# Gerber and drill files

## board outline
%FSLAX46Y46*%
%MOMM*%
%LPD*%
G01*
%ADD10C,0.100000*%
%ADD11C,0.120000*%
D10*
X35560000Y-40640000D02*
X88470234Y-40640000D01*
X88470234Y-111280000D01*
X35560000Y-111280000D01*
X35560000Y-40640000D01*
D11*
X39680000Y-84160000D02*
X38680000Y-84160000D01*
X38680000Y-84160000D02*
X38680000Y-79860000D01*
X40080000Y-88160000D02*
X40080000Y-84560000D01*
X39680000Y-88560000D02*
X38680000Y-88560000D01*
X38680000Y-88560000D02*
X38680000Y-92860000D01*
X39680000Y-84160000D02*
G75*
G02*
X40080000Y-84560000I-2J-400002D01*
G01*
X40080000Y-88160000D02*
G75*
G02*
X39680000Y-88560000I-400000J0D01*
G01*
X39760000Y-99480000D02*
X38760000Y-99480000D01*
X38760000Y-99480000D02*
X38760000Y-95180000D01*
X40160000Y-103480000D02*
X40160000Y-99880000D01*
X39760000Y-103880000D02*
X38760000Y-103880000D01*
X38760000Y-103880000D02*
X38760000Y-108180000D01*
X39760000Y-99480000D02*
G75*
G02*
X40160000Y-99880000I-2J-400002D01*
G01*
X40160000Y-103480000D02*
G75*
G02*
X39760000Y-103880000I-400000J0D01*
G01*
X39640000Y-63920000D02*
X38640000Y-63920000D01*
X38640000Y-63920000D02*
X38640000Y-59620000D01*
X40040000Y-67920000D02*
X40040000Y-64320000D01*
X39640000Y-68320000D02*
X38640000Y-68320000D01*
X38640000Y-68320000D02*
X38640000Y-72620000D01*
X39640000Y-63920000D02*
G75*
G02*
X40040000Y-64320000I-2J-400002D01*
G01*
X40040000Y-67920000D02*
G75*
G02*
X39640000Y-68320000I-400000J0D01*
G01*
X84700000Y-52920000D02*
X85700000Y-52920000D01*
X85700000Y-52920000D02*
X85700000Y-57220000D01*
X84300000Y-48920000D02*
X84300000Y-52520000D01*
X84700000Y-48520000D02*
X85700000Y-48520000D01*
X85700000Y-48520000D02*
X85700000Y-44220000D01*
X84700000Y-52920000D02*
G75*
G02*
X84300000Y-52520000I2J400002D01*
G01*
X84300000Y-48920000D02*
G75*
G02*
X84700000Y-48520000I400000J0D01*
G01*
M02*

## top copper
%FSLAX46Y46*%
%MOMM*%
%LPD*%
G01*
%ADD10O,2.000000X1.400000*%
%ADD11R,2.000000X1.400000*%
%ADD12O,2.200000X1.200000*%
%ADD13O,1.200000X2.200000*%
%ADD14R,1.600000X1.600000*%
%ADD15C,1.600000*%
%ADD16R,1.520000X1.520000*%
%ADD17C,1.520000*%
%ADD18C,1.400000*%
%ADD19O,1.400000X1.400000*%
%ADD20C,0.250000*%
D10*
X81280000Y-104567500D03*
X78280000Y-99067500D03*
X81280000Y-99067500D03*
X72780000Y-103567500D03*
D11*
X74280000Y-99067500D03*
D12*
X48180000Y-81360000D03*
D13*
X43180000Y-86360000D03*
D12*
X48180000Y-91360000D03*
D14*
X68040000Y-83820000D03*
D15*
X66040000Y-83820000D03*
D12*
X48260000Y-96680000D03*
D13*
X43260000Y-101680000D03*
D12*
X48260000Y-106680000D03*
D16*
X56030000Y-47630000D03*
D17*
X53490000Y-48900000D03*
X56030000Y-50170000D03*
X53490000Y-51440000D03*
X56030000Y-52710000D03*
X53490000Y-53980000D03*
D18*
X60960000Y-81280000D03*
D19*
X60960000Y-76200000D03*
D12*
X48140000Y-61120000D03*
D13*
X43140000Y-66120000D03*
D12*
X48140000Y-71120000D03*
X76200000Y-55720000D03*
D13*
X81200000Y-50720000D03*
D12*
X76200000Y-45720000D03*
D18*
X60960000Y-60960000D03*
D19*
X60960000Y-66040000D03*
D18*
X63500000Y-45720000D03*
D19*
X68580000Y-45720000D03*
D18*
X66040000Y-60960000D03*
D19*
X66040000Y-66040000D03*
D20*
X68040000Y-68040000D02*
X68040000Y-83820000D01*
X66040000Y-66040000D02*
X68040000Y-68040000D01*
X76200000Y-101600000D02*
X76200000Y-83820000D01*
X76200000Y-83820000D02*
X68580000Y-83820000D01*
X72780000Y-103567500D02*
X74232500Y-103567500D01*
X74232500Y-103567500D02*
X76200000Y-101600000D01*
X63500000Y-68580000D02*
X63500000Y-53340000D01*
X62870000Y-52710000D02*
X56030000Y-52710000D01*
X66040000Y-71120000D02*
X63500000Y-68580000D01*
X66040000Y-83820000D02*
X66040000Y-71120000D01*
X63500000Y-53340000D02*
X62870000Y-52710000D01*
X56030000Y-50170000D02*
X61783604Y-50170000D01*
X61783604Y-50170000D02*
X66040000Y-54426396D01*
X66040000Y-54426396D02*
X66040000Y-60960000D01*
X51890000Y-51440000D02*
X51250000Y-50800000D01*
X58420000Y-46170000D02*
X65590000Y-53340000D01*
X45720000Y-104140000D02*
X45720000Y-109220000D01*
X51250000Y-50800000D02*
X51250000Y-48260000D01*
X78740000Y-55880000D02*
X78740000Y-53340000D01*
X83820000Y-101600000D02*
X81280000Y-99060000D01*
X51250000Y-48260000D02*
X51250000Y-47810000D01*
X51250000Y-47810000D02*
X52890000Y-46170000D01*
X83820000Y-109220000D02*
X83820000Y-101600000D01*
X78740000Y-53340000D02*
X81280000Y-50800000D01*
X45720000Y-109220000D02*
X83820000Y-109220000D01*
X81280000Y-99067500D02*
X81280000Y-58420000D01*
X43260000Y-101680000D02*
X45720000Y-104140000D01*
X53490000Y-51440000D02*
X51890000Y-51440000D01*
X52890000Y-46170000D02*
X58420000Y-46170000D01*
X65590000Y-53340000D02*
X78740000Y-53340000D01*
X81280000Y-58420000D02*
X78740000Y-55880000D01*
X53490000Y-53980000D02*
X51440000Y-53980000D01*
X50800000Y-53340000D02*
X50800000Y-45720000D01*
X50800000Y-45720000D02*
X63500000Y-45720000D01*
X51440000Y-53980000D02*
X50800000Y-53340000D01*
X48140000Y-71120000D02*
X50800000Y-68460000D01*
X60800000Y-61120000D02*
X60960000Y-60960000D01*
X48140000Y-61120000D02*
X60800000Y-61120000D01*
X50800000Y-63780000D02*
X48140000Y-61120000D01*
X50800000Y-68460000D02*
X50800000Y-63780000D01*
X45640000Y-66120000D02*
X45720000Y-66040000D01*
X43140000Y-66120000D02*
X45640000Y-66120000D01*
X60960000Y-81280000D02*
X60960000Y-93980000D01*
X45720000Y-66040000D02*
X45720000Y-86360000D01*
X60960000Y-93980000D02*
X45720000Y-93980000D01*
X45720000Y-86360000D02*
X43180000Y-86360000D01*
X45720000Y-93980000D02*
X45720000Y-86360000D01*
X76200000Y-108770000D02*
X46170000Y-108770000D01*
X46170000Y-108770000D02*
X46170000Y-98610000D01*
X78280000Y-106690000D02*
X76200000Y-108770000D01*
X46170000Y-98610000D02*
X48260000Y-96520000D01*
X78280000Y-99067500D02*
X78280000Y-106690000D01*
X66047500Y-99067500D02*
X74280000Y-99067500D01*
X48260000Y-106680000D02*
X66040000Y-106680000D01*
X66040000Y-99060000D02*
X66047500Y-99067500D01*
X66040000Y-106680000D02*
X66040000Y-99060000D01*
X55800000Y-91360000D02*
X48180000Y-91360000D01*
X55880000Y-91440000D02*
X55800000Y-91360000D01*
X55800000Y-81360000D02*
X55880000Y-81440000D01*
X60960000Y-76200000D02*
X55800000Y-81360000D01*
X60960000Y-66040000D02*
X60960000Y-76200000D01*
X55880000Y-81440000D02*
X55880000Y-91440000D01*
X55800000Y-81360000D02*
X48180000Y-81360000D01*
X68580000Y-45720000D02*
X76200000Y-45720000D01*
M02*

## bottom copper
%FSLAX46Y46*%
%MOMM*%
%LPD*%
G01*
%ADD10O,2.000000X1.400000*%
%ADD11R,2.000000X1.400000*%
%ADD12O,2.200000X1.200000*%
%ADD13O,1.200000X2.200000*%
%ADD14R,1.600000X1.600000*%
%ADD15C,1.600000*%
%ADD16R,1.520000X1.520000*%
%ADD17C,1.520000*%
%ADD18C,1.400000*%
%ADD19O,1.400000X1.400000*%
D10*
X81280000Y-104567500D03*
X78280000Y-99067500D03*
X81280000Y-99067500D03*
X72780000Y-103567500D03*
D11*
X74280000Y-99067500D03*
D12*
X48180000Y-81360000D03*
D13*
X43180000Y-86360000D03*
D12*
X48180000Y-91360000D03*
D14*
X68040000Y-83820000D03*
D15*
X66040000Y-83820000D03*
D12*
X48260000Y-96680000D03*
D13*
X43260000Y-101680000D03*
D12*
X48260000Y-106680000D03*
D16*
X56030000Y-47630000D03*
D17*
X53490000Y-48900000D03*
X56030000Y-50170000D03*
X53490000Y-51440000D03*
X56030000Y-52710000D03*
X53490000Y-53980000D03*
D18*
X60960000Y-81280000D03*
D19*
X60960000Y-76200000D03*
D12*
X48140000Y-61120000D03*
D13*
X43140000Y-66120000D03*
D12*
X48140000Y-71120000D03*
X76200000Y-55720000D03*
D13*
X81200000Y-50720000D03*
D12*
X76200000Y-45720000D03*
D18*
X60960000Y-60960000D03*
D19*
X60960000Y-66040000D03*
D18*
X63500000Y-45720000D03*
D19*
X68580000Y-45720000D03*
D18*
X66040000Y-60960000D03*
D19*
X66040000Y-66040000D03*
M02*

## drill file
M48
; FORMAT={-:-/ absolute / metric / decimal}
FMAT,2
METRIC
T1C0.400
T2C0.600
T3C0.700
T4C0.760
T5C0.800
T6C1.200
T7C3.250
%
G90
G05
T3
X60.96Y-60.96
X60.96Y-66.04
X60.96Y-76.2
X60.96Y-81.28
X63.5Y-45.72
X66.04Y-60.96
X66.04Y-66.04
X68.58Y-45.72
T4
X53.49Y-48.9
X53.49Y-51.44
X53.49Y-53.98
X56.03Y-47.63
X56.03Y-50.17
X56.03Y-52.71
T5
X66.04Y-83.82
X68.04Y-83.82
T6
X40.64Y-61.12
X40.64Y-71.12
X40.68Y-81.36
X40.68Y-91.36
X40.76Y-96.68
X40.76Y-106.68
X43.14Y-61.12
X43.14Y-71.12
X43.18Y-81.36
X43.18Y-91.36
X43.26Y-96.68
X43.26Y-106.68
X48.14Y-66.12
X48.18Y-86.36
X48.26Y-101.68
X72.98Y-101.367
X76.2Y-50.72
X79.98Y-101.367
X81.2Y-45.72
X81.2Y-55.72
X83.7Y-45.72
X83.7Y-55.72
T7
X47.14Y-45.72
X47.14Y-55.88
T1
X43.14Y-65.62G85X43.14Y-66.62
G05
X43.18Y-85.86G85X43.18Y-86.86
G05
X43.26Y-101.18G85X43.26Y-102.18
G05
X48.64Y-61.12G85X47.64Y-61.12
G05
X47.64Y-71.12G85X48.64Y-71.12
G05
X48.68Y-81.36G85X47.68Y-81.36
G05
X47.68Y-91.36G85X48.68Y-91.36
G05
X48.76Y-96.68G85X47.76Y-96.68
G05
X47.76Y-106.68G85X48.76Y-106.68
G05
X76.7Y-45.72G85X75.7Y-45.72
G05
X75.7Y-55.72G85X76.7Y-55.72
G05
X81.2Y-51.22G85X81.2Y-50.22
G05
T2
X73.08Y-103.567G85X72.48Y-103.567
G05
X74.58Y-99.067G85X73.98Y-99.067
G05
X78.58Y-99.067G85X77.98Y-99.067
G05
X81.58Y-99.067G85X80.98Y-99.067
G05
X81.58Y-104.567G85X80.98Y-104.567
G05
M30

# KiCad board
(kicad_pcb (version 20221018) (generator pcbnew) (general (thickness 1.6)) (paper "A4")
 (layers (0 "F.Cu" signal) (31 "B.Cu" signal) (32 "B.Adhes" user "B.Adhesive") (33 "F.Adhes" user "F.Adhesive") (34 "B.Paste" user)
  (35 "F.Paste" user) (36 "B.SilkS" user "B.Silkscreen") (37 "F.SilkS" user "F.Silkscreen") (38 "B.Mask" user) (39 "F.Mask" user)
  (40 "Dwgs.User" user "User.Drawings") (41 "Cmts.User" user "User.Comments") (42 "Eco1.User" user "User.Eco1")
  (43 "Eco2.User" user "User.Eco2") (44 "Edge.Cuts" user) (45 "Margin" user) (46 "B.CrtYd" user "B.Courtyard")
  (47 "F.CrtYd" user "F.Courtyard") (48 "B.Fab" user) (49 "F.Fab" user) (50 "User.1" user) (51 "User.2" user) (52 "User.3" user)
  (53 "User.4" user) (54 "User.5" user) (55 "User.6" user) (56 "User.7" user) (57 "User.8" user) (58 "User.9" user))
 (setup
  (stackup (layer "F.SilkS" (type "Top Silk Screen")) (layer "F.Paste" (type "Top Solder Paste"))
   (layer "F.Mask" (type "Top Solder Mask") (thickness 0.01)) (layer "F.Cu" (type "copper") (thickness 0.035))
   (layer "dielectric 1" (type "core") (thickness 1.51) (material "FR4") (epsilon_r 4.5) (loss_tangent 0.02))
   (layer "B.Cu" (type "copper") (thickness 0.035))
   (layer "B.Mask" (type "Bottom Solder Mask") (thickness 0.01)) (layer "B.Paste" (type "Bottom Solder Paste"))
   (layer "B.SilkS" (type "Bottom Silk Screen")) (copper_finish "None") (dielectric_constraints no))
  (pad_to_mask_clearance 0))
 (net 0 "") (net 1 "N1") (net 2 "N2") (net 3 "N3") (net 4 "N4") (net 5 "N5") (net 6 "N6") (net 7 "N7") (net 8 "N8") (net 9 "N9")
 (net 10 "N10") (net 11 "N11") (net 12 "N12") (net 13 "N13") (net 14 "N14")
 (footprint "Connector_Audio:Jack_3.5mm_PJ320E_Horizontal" (layer "F.Cu") (at 74.28 99.0675 -90)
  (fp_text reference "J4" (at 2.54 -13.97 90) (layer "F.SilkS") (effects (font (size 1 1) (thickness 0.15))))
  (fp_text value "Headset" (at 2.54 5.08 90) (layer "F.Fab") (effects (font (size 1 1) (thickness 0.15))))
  (pad "" np_thru_hole circle (at 2.3 -5.7 180) (size 1.2 1.2) (drill 1.2) (layers "*.Cu" "*.Mask"))
  (pad "" np_thru_hole circle (at 2.3 1.3 180) (size 1.2 1.2) (drill 1.2) (layers "*.Cu" "*.Mask"))
  (pad "" thru_hole oval (at 5.5 -7 180) (size 2 1.4) (drill oval 1.2 0.6) (layers "*.Cu" "*.Mask"))
  (pad "R1" thru_hole oval (at 0 -4 180) (size 2 1.4) (drill oval 1.2 0.6) (layers "*.Cu" "*.Mask") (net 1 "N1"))
  (pad "R2" thru_hole oval (at 0 -7 180) (size 2 1.4) (drill oval 1.2 0.6) (layers "*.Cu" "*.Mask") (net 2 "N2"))
  (pad "S" thru_hole oval (at 4.5 1.5 180) (size 2 1.4) (drill oval 1.2 0.6) (layers "*.Cu" "*.Mask") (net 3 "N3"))
  (pad "T" thru_hole rect (at 0 0 180) (size 2 1.4) (drill oval 1.2 0.6) (layers "*.Cu" "*.Mask") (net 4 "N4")))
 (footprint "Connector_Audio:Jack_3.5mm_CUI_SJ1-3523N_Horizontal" (layer "F.Cu") (at 43.18 86.36 -90)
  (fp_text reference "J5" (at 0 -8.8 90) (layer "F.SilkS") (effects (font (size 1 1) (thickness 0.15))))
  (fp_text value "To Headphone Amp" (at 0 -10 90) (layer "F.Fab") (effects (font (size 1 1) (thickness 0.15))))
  (fp_line (start -2.2 3.5) (end -2.2 4.5) (stroke (width 0.12) (type solid)) (layer "Edge.Cuts"))
  (fp_line (start -2.2 4.5) (end -6.5 4.5) (stroke (width 0.12) (type solid)) (layer "Edge.Cuts"))
  (fp_line (start 1.8 3.1) (end -1.8 3.1) (stroke (width 0.12) (type solid)) (layer "Edge.Cuts"))
  (fp_line (start 2.2 3.5) (end 2.2 4.5) (stroke (width 0.12) (type solid)) (layer "Edge.Cuts"))
  (fp_line (start 2.2 4.5) (end 6.5 4.5) (stroke (width 0.12) (type solid)) (layer "Edge.Cuts"))
  (fp_arc (start -2.2 3.5) (mid -2.082842 3.217158) (end -1.8 3.1) (stroke (width 0.12) (type solid)) (layer "Edge.Cuts"))
  (fp_arc (start 1.8 3.1) (mid 2.082843 3.217157) (end 2.2 3.5) (stroke (width 0.12) (type solid)) (layer "Edge.Cuts"))
  (pad "" np_thru_hole circle (at -5 0 270) (size 1.2 1.2) (drill 1.2) (layers "*.Cu"))
  (pad "" np_thru_hole circle (at -5 2.5 270) (size 1.2 1.2) (drill 1.2) (layers "*.Cu"))
  (pad "" np_thru_hole circle (at 0 -5 270) (size 1.2 1.2) (drill 1.2) (layers "*.Cu"))
  (pad "" np_thru_hole circle (at 5 0 270) (size 1.2 1.2) (drill 1.2) (layers "*.Cu"))
  (pad "" np_thru_hole circle (at 5 2.5 270) (size 1.2 1.2) (drill 1.2) (layers "*.Cu"))
  (pad "R" thru_hole oval (at -5 -5 270) (size 1.2 2.2) (drill oval 0.4 1.4) (layers "*.Cu" "*.Mask") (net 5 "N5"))
  (pad "S" thru_hole oval (at 0 0 270) (size 2.2 1.2) (drill oval 1.4 0.4) (layers "*.Cu" "*.Mask") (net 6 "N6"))
  (pad "T" thru_hole oval (at 5 -5 90) (size 1.2 2.2) (drill oval 0.4 1.4) (layers "*.Cu" "*.Mask") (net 5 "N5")))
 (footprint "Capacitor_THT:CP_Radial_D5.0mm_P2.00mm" (layer "F.Cu") (at 68.04 83.82 180)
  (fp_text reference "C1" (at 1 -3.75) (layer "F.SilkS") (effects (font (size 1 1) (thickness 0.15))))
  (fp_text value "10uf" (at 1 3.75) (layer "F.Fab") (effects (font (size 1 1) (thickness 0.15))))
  (pad "1" thru_hole rect (at 0 0 180) (size 1.6 1.6) (drill 0.8) (layers "*.Cu" "*.Mask") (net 3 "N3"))
  (pad "2" thru_hole circle (at 2 0 180) (size 1.6 1.6) (drill 0.8) (layers "*.Cu" "*.Mask") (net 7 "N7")))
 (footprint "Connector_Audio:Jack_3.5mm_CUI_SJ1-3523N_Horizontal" (layer "F.Cu") (at 43.26 101.68 -90)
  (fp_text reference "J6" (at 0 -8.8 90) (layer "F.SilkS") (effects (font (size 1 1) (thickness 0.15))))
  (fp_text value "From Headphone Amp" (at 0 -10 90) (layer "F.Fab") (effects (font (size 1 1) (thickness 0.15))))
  (fp_line (start -2.2 3.5) (end -2.2 4.5) (stroke (width 0.12) (type solid)) (layer "Edge.Cuts"))
  (fp_line (start -2.2 4.5) (end -6.5 4.5) (stroke (width 0.12) (type solid)) (layer "Edge.Cuts"))
  (fp_line (start 1.8 3.1) (end -1.8 3.1) (stroke (width 0.12) (type solid)) (layer "Edge.Cuts"))
  (fp_line (start 2.2 3.5) (end 2.2 4.5) (stroke (width 0.12) (type solid)) (layer "Edge.Cuts"))
  (fp_line (start 2.2 4.5) (end 6.5 4.5) (stroke (width 0.12) (type solid)) (layer "Edge.Cuts"))
  (fp_arc (start -2.2 3.5) (mid -2.082842 3.217158) (end -1.8 3.1) (stroke (width 0.12) (type solid)) (layer "Edge.Cuts"))
  (fp_arc (start 1.8 3.1) (mid 2.082843 3.217157) (end 2.2 3.5) (stroke (width 0.12) (type solid)) (layer "Edge.Cuts"))
  (pad "" np_thru_hole circle (at -5 0 270) (size 1.2 1.2) (drill 1.2) (layers "*.Cu"))
  (pad "" np_thru_hole circle (at -5 2.5 270) (size 1.2 1.2) (drill 1.2) (layers "*.Cu"))
  (pad "" np_thru_hole circle (at 0 -5 270) (size 1.2 1.2) (drill 1.2) (layers "*.Cu"))
  (pad "" np_thru_hole circle (at 5 0 270) (size 1.2 1.2) (drill 1.2) (layers "*.Cu"))
  (pad "" np_thru_hole circle (at 5 2.5 270) (size 1.2 1.2) (drill 1.2) (layers "*.Cu"))
  (pad "R" thru_hole oval (at -5 -5 270) (size 1.2 2.2) (drill oval 0.4 1.4) (layers "*.Cu" "*.Mask") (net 1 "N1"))
  (pad "S" thru_hole oval (at 0 0 270) (size 2.2 1.2) (drill oval 1.4 0.4) (layers "*.Cu" "*.Mask") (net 2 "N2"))
  (pad "T" thru_hole oval (at 5 -5 90) (size 1.2 2.2) (drill oval 0.4 1.4) (layers "*.Cu" "*.Mask") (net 4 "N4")))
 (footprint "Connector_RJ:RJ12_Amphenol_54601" (layer "F.Cu") (at 56.03 47.63 -90)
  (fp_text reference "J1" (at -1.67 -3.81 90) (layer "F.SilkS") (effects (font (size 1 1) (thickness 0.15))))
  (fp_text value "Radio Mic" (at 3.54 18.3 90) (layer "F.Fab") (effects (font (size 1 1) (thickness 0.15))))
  (pad "" np_thru_hole circle (at -1.91 8.89 270) (size 3.25 3.25) (drill 3.25) (layers "*.Cu" "*.Mask"))
  (pad "" np_thru_hole circle (at 8.25 8.89 270) (size 3.25 3.25) (drill 3.25) (layers "*.Cu" "*.Mask"))
  (pad "1" thru_hole rect (at 0 0 270) (size 1.52 1.52) (drill 0.76) (layers "*.Cu" "*.Mask") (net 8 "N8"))
  (pad "2" thru_hole circle (at 1.27 2.54 270) (size 1.52 1.52) (drill 0.76) (layers "*.Cu" "*.Mask") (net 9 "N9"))
  (pad "3" thru_hole circle (at 2.54 0 270) (size 1.52 1.52) (drill 0.76) (layers "*.Cu" "*.Mask") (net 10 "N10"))
  (pad "4" thru_hole circle (at 3.81 2.54 270) (size 1.52 1.52) (drill 0.76) (layers "*.Cu" "*.Mask") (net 2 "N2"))
  (pad "5" thru_hole circle (at 5.08 0 270) (size 1.52 1.52) (drill 0.76) (layers "*.Cu" "*.Mask") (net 7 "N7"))
  (pad "6" thru_hole circle (at 6.35 2.54 270) (size 1.52 1.52) (drill 0.76) (layers "*.Cu" "*.Mask") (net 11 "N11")))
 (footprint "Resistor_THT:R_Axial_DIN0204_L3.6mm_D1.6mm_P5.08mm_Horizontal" (layer "F.Cu") (at 60.96 81.28 90)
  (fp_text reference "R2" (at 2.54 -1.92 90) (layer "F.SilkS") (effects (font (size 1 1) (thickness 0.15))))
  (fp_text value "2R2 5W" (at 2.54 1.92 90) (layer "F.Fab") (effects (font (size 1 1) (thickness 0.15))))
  (pad "1" thru_hole circle (at 0 0 90) (size 1.4 1.4) (drill 0.7) (layers "*.Cu" "*.Mask") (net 6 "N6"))
  (pad "2" thru_hole oval (at 5.08 0 90) (size 1.4 1.4) (drill 0.7) (layers "*.Cu" "*.Mask") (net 5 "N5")))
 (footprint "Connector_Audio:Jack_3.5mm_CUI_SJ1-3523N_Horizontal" (layer "F.Cu") (at 43.14 66.12 -90)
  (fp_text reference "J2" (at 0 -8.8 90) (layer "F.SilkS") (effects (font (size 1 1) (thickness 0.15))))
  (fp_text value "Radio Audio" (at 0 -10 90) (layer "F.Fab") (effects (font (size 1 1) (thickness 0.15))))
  (fp_line (start -2.2 3.5) (end -2.2 4.5) (stroke (width 0.12) (type solid)) (layer "Edge.Cuts"))
  (fp_line (start -2.2 4.5) (end -6.5 4.5) (stroke (width 0.12) (type solid)) (layer "Edge.Cuts"))
  (fp_line (start 1.8 3.1) (end -1.8 3.1) (stroke (width 0.12) (type solid)) (layer "Edge.Cuts"))
  (fp_line (start 2.2 3.5) (end 2.2 4.5) (stroke (width 0.12) (type solid)) (layer "Edge.Cuts"))
  (fp_line (start 2.2 4.5) (end 6.5 4.5) (stroke (width 0.12) (type solid)) (layer "Edge.Cuts"))
  (fp_arc (start -2.2 3.5) (mid -2.082842 3.217158) (end -1.8 3.1) (stroke (width 0.12) (type solid)) (layer "Edge.Cuts"))
  (fp_arc (start 1.8 3.1) (mid 2.082843 3.217157) (end 2.2 3.5) (stroke (width 0.12) (type solid)) (layer "Edge.Cuts"))
  (pad "" np_thru_hole circle (at -5 0 270) (size 1.2 1.2) (drill 1.2) (layers "*.Cu"))
  (pad "" np_thru_hole circle (at -5 2.5 270) (size 1.2 1.2) (drill 1.2) (layers "*.Cu"))
  (pad "" np_thru_hole circle (at 0 -5 270) (size 1.2 1.2) (drill 1.2) (layers "*.Cu"))
  (pad "" np_thru_hole circle (at 5 0 270) (size 1.2 1.2) (drill 1.2) (layers "*.Cu"))
  (pad "" np_thru_hole circle (at 5 2.5 270) (size 1.2 1.2) (drill 1.2) (layers "*.Cu"))
  (pad "R" thru_hole oval (at -5 -5 270) (size 1.2 2.2) (drill oval 0.4 1.4) (layers "*.Cu" "*.Mask") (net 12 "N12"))
  (pad "S" thru_hole oval (at 0 0 270) (size 2.2 1.2) (drill oval 1.4 0.4) (layers "*.Cu" "*.Mask") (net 6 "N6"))
  (pad "T" thru_hole oval (at 5 -5 90) (size 1.2 2.2) (drill oval 0.4 1.4) (layers "*.Cu" "*.Mask") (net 12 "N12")))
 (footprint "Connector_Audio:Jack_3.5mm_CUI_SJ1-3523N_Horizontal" (layer "F.Cu") (at 81.2 50.72 90)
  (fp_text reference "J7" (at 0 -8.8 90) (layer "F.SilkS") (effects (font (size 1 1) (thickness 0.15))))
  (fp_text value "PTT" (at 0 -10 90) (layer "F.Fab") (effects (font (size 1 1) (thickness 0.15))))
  (fp_line (start -2.2 3.5) (end -2.2 4.5) (stroke (width 0.12) (type solid)) (layer "Edge.Cuts"))
  (fp_line (start -2.2 4.5) (end -6.5 4.5) (stroke (width 0.12) (type solid)) (layer "Edge.Cuts"))
  (fp_line (start 1.8 3.1) (end -1.8 3.1) (stroke (width 0.12) (type solid)) (layer "Edge.Cuts"))
  (fp_line (start 2.2 3.5) (end 2.2 4.5) (stroke (width 0.12) (type solid)) (layer "Edge.Cuts"))
  (fp_line (start 2.2 4.5) (end 6.5 4.5) (stroke (width 0.12) (type solid)) (layer "Edge.Cuts"))
  (fp_arc (start -2.2 3.5) (mid -2.082842 3.217158) (end -1.8 3.1) (stroke (width 0.12) (type solid)) (layer "Edge.Cuts"))
  (fp_arc (start 1.8 3.1) (mid 2.082843 3.217157) (end 2.2 3.5) (stroke (width 0.12) (type solid)) (layer "Edge.Cuts"))
  (pad "" np_thru_hole circle (at -5 0 90) (size 1.2 1.2) (drill 1.2) (layers "*.Cu"))
  (pad "" np_thru_hole circle (at -5 2.5 90) (size 1.2 1.2) (drill 1.2) (layers "*.Cu"))
  (pad "" np_thru_hole circle (at 0 -5 90) (size 1.2 1.2) (drill 1.2) (layers "*.Cu"))
  (pad "" np_thru_hole circle (at 5 0 90) (size 1.2 1.2) (drill 1.2) (layers "*.Cu"))
  (pad "" np_thru_hole circle (at 5 2.5 90) (size 1.2 1.2) (drill 1.2) (layers "*.Cu"))
  (pad "R" thru_hole oval (at -5 -5 90) (size 1.2 2.2) (drill oval 0.4 1.4) (layers "*.Cu" "*.Mask") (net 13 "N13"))
  (pad "S" thru_hole oval (at 0 0 90) (size 2.2 1.2) (drill oval 1.4 0.4) (layers "*.Cu" "*.Mask") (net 2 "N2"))
  (pad "T" thru_hole oval (at 5 -5 270) (size 1.2 2.2) (drill oval 0.4 1.4) (layers "*.Cu" "*.Mask") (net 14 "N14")))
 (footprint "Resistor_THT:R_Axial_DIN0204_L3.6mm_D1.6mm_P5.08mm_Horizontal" (layer "F.Cu") (at 60.96 60.96 -90)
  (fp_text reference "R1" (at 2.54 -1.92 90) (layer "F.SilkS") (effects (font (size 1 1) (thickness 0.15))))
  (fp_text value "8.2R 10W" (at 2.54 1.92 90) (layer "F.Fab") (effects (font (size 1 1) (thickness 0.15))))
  (pad "1" thru_hole circle (at 0 0 270) (size 1.4 1.4) (drill 0.7) (layers "*.Cu" "*.Mask") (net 12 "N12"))
  (pad "2" thru_hole oval (at 5.08 0 270) (size 1.4 1.4) (drill 0.7) (layers "*.Cu" "*.Mask") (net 5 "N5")))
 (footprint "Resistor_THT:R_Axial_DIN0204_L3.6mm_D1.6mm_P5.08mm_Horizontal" (layer "F.Cu") (at 63.5 45.72)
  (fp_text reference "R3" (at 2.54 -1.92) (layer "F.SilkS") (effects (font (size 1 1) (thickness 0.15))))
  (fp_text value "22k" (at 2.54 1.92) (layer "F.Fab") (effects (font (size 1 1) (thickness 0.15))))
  (pad "1" thru_hole circle (at 0 0) (size 1.4 1.4) (drill 0.7) (layers "*.Cu" "*.Mask") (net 11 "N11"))
  (pad "2" thru_hole oval (at 5.08 0) (size 1.4 1.4) (drill 0.7) (layers "*.Cu" "*.Mask") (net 14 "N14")))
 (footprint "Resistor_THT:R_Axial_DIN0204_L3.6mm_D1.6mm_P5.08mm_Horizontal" (layer "F.Cu") (at 66.04 60.96 -90)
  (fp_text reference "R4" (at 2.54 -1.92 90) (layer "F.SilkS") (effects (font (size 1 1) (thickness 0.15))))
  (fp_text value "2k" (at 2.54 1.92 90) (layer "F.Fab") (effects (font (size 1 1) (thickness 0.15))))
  (pad "1" thru_hole circle (at 0 0 270) (size 1.4 1.4) (drill 0.7) (layers "*.Cu" "*.Mask") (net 10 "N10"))
  (pad "2" thru_hole oval (at 5.08 0 270) (size 1.4 1.4) (drill 0.7) (layers "*.Cu" "*.Mask") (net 3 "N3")))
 (gr_rect (start 35.56 40.64) (end 88.470234 111.28) (stroke (width 0.1) (type default)) (fill none) (layer "Edge.Cuts"))
 (segment (start 68.04 68.04) (end 68.04 83.82) (width 0.25) (layer "F.Cu") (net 3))
 (segment (start 66.04 66.04) (end 68.04 68.04) (width 0.25) (layer "F.Cu") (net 3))
 (segment (start 76.2 101.6) (end 76.2 83.82) (width 0.25) (layer "F.Cu") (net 3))
 (segment (start 76.2 83.82) (end 68.58 83.82) (width 0.25) (layer "F.Cu") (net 3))
 (segment (start 72.78 103.5675) (end 74.2325 103.5675) (width 0.25) (layer "F.Cu") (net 3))
 (segment (start 74.2325 103.5675) (end 76.2 101.6) (width 0.25) (layer "F.Cu") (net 3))
 (segment (start 63.5 68.58) (end 63.5 53.34) (width 0.25) (layer "F.Cu") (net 7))
 (segment (start 62.87 52.71) (end 56.03 52.71) (width 0.25) (layer "F.Cu") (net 7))
 (segment (start 66.04 71.12) (end 63.5 68.58) (width 0.25) (layer "F.Cu") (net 7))
 (segment (start 66.04 83.82) (end 66.04 71.12) (width 0.25) (layer "F.Cu") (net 7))
 (segment (start 63.5 53.34) (end 62.87 52.71) (width 0.25) (layer "F.Cu") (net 7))
 (segment (start 56.03 50.17) (end 61.783604 50.17) (width 0.25) (layer "F.Cu") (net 10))
 (segment (start 61.783604 50.17) (end 66.04 54.426396) (width 0.25) (layer "F.Cu") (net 10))
 (segment (start 66.04 54.426396) (end 66.04 60.96) (width 0.25) (layer "F.Cu") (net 10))
 (segment (start 51.89 51.44) (end 51.25 50.8) (width 0.25) (layer "F.Cu") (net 2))
 (segment (start 58.42 46.17) (end 65.59 53.34) (width 0.25) (layer "F.Cu") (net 2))
 (segment (start 45.72 104.14) (end 45.72 109.22) (width 0.25) (layer "F.Cu") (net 2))
 (segment (start 51.25 50.8) (end 51.25 48.26) (width 0.25) (layer "F.Cu") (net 2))
 (segment (start 78.74 55.88) (end 78.74 53.34) (width 0.25) (layer "F.Cu") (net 2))
 (segment (start 83.82 101.6) (end 81.28 99.06) (width 0.25) (layer "F.Cu") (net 2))
 (segment (start 51.25 48.26) (end 51.25 47.81) (width 0.25) (layer "F.Cu") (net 2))
 (segment (start 51.25 47.81) (end 52.89 46.17) (width 0.25) (layer "F.Cu") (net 2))
 (segment (start 83.82 109.22) (end 83.82 101.6) (width 0.25) (layer "F.Cu") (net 2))
 (segment (start 78.74 53.34) (end 81.28 50.8) (width 0.25) (layer "F.Cu") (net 2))
 (segment (start 45.72 109.22) (end 83.82 109.22) (width 0.25) (layer "F.Cu") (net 2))
 (segment (start 81.28 99.0675) (end 81.28 58.42) (width 0.25) (layer "F.Cu") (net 2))
 (segment (start 43.26 101.68) (end 45.72 104.14) (width 0.25) (layer "F.Cu") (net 2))
 (segment (start 53.49 51.44) (end 51.89 51.44) (width 0.25) (layer "F.Cu") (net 2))
 (segment (start 52.89 46.17) (end 58.42 46.17) (width 0.25) (layer "F.Cu") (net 2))
 (segment (start 65.59 53.34) (end 78.74 53.34) (width 0.25) (layer "F.Cu") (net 2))
 (segment (start 81.28 58.42) (end 78.74 55.88) (width 0.25) (layer "F.Cu") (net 2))
 (segment (start 53.49 53.98) (end 51.44 53.98) (width 0.25) (layer "F.Cu") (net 11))
 (segment (start 50.8 53.34) (end 50.8 45.72) (width 0.25) (layer "F.Cu") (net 11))
 (segment (start 50.8 45.72) (end 63.5 45.72) (width 0.25) (layer "F.Cu") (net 11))
 (segment (start 51.44 53.98) (end 50.8 53.34) (width 0.25) (layer "F.Cu") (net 11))
 (segment (start 48.14 71.12) (end 50.8 68.46) (width 0.25) (layer "F.Cu") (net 12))
 (segment (start 60.8 61.12) (end 60.96 60.96) (width 0.25) (layer "F.Cu") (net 12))
 (segment (start 48.14 61.12) (end 60.8 61.12) (width 0.25) (layer "F.Cu") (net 12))
 (segment (start 50.8 63.78) (end 48.14 61.12) (width 0.25) (layer "F.Cu") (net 12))
 (segment (start 50.8 68.46) (end 50.8 63.78) (width 0.25) (layer "F.Cu") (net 12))
 (segment (start 45.64 66.12) (end 45.72 66.04) (width 0.25) (layer "F.Cu") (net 6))
 (segment (start 43.14 66.12) (end 45.64 66.12) (width 0.25) (layer "F.Cu") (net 6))
 (segment (start 60.96 81.28) (end 60.96 93.98) (width 0.25) (layer "F.Cu") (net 6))
 (segment (start 45.72 66.04) (end 45.72 86.36) (width 0.25) (layer "F.Cu") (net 6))
 (segment (start 60.96 93.98) (end 45.72 93.98) (width 0.25) (layer "F.Cu") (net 6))
 (segment (start 45.72 86.36) (end 43.18 86.36) (width 0.25) (layer "F.Cu") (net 6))
 (segment (start 45.72 93.98) (end 45.72 86.36) (width 0.25) (layer "F.Cu") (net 6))
 (segment (start 76.2 108.77) (end 46.17 108.77) (width 0.25) (layer "F.Cu") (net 1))
 (segment (start 46.17 108.77) (end 46.17 98.61) (width 0.25) (layer "F.Cu") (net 1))
 (segment (start 78.28 106.69) (end 76.2 108.77) (width 0.25) (layer "F.Cu") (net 1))
 (segment (start 46.17 98.61) (end 48.26 96.52) (width 0.25) (layer "F.Cu") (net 1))
 (segment (start 78.28 99.0675) (end 78.28 106.69) (width 0.25) (layer "F.Cu") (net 1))
 (segment (start 66.0475 99.0675) (end 74.28 99.0675) (width 0.25) (layer "F.Cu") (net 4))
 (segment (start 48.26 106.68) (end 66.04 106.68) (width 0.25) (layer "F.Cu") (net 4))
 (segment (start 66.04 99.06) (end 66.0475 99.0675) (width 0.25) (layer "F.Cu") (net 4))
 (segment (start 66.04 106.68) (end 66.04 99.06) (width 0.25) (layer "F.Cu") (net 4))
 (segment (start 55.8 91.36) (end 48.18 91.36) (width 0.25) (layer "F.Cu") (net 5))
 (segment (start 55.88 91.44) (end 55.8 91.36) (width 0.25) (layer "F.Cu") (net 5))
 (segment (start 55.8 81.36) (end 55.88 81.44) (width 0.25) (layer "F.Cu") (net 5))
 (segment (start 60.96 76.2) (end 55.8 81.36) (width 0.25) (layer "F.Cu") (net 5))
 (segment (start 60.96 66.04) (end 60.96 76.2) (width 0.25) (layer "F.Cu") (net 5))
 (segment (start 55.88 81.44) (end 55.88 91.44) (width 0.25) (layer "F.Cu") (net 5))
 (segment (start 55.8 81.36) (end 48.18 81.36) (width 0.25) (layer "F.Cu") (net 5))
 (segment (start 68.58 45.72) (end 76.2 45.72) (width 0.25) (layer "F.Cu") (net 14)))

